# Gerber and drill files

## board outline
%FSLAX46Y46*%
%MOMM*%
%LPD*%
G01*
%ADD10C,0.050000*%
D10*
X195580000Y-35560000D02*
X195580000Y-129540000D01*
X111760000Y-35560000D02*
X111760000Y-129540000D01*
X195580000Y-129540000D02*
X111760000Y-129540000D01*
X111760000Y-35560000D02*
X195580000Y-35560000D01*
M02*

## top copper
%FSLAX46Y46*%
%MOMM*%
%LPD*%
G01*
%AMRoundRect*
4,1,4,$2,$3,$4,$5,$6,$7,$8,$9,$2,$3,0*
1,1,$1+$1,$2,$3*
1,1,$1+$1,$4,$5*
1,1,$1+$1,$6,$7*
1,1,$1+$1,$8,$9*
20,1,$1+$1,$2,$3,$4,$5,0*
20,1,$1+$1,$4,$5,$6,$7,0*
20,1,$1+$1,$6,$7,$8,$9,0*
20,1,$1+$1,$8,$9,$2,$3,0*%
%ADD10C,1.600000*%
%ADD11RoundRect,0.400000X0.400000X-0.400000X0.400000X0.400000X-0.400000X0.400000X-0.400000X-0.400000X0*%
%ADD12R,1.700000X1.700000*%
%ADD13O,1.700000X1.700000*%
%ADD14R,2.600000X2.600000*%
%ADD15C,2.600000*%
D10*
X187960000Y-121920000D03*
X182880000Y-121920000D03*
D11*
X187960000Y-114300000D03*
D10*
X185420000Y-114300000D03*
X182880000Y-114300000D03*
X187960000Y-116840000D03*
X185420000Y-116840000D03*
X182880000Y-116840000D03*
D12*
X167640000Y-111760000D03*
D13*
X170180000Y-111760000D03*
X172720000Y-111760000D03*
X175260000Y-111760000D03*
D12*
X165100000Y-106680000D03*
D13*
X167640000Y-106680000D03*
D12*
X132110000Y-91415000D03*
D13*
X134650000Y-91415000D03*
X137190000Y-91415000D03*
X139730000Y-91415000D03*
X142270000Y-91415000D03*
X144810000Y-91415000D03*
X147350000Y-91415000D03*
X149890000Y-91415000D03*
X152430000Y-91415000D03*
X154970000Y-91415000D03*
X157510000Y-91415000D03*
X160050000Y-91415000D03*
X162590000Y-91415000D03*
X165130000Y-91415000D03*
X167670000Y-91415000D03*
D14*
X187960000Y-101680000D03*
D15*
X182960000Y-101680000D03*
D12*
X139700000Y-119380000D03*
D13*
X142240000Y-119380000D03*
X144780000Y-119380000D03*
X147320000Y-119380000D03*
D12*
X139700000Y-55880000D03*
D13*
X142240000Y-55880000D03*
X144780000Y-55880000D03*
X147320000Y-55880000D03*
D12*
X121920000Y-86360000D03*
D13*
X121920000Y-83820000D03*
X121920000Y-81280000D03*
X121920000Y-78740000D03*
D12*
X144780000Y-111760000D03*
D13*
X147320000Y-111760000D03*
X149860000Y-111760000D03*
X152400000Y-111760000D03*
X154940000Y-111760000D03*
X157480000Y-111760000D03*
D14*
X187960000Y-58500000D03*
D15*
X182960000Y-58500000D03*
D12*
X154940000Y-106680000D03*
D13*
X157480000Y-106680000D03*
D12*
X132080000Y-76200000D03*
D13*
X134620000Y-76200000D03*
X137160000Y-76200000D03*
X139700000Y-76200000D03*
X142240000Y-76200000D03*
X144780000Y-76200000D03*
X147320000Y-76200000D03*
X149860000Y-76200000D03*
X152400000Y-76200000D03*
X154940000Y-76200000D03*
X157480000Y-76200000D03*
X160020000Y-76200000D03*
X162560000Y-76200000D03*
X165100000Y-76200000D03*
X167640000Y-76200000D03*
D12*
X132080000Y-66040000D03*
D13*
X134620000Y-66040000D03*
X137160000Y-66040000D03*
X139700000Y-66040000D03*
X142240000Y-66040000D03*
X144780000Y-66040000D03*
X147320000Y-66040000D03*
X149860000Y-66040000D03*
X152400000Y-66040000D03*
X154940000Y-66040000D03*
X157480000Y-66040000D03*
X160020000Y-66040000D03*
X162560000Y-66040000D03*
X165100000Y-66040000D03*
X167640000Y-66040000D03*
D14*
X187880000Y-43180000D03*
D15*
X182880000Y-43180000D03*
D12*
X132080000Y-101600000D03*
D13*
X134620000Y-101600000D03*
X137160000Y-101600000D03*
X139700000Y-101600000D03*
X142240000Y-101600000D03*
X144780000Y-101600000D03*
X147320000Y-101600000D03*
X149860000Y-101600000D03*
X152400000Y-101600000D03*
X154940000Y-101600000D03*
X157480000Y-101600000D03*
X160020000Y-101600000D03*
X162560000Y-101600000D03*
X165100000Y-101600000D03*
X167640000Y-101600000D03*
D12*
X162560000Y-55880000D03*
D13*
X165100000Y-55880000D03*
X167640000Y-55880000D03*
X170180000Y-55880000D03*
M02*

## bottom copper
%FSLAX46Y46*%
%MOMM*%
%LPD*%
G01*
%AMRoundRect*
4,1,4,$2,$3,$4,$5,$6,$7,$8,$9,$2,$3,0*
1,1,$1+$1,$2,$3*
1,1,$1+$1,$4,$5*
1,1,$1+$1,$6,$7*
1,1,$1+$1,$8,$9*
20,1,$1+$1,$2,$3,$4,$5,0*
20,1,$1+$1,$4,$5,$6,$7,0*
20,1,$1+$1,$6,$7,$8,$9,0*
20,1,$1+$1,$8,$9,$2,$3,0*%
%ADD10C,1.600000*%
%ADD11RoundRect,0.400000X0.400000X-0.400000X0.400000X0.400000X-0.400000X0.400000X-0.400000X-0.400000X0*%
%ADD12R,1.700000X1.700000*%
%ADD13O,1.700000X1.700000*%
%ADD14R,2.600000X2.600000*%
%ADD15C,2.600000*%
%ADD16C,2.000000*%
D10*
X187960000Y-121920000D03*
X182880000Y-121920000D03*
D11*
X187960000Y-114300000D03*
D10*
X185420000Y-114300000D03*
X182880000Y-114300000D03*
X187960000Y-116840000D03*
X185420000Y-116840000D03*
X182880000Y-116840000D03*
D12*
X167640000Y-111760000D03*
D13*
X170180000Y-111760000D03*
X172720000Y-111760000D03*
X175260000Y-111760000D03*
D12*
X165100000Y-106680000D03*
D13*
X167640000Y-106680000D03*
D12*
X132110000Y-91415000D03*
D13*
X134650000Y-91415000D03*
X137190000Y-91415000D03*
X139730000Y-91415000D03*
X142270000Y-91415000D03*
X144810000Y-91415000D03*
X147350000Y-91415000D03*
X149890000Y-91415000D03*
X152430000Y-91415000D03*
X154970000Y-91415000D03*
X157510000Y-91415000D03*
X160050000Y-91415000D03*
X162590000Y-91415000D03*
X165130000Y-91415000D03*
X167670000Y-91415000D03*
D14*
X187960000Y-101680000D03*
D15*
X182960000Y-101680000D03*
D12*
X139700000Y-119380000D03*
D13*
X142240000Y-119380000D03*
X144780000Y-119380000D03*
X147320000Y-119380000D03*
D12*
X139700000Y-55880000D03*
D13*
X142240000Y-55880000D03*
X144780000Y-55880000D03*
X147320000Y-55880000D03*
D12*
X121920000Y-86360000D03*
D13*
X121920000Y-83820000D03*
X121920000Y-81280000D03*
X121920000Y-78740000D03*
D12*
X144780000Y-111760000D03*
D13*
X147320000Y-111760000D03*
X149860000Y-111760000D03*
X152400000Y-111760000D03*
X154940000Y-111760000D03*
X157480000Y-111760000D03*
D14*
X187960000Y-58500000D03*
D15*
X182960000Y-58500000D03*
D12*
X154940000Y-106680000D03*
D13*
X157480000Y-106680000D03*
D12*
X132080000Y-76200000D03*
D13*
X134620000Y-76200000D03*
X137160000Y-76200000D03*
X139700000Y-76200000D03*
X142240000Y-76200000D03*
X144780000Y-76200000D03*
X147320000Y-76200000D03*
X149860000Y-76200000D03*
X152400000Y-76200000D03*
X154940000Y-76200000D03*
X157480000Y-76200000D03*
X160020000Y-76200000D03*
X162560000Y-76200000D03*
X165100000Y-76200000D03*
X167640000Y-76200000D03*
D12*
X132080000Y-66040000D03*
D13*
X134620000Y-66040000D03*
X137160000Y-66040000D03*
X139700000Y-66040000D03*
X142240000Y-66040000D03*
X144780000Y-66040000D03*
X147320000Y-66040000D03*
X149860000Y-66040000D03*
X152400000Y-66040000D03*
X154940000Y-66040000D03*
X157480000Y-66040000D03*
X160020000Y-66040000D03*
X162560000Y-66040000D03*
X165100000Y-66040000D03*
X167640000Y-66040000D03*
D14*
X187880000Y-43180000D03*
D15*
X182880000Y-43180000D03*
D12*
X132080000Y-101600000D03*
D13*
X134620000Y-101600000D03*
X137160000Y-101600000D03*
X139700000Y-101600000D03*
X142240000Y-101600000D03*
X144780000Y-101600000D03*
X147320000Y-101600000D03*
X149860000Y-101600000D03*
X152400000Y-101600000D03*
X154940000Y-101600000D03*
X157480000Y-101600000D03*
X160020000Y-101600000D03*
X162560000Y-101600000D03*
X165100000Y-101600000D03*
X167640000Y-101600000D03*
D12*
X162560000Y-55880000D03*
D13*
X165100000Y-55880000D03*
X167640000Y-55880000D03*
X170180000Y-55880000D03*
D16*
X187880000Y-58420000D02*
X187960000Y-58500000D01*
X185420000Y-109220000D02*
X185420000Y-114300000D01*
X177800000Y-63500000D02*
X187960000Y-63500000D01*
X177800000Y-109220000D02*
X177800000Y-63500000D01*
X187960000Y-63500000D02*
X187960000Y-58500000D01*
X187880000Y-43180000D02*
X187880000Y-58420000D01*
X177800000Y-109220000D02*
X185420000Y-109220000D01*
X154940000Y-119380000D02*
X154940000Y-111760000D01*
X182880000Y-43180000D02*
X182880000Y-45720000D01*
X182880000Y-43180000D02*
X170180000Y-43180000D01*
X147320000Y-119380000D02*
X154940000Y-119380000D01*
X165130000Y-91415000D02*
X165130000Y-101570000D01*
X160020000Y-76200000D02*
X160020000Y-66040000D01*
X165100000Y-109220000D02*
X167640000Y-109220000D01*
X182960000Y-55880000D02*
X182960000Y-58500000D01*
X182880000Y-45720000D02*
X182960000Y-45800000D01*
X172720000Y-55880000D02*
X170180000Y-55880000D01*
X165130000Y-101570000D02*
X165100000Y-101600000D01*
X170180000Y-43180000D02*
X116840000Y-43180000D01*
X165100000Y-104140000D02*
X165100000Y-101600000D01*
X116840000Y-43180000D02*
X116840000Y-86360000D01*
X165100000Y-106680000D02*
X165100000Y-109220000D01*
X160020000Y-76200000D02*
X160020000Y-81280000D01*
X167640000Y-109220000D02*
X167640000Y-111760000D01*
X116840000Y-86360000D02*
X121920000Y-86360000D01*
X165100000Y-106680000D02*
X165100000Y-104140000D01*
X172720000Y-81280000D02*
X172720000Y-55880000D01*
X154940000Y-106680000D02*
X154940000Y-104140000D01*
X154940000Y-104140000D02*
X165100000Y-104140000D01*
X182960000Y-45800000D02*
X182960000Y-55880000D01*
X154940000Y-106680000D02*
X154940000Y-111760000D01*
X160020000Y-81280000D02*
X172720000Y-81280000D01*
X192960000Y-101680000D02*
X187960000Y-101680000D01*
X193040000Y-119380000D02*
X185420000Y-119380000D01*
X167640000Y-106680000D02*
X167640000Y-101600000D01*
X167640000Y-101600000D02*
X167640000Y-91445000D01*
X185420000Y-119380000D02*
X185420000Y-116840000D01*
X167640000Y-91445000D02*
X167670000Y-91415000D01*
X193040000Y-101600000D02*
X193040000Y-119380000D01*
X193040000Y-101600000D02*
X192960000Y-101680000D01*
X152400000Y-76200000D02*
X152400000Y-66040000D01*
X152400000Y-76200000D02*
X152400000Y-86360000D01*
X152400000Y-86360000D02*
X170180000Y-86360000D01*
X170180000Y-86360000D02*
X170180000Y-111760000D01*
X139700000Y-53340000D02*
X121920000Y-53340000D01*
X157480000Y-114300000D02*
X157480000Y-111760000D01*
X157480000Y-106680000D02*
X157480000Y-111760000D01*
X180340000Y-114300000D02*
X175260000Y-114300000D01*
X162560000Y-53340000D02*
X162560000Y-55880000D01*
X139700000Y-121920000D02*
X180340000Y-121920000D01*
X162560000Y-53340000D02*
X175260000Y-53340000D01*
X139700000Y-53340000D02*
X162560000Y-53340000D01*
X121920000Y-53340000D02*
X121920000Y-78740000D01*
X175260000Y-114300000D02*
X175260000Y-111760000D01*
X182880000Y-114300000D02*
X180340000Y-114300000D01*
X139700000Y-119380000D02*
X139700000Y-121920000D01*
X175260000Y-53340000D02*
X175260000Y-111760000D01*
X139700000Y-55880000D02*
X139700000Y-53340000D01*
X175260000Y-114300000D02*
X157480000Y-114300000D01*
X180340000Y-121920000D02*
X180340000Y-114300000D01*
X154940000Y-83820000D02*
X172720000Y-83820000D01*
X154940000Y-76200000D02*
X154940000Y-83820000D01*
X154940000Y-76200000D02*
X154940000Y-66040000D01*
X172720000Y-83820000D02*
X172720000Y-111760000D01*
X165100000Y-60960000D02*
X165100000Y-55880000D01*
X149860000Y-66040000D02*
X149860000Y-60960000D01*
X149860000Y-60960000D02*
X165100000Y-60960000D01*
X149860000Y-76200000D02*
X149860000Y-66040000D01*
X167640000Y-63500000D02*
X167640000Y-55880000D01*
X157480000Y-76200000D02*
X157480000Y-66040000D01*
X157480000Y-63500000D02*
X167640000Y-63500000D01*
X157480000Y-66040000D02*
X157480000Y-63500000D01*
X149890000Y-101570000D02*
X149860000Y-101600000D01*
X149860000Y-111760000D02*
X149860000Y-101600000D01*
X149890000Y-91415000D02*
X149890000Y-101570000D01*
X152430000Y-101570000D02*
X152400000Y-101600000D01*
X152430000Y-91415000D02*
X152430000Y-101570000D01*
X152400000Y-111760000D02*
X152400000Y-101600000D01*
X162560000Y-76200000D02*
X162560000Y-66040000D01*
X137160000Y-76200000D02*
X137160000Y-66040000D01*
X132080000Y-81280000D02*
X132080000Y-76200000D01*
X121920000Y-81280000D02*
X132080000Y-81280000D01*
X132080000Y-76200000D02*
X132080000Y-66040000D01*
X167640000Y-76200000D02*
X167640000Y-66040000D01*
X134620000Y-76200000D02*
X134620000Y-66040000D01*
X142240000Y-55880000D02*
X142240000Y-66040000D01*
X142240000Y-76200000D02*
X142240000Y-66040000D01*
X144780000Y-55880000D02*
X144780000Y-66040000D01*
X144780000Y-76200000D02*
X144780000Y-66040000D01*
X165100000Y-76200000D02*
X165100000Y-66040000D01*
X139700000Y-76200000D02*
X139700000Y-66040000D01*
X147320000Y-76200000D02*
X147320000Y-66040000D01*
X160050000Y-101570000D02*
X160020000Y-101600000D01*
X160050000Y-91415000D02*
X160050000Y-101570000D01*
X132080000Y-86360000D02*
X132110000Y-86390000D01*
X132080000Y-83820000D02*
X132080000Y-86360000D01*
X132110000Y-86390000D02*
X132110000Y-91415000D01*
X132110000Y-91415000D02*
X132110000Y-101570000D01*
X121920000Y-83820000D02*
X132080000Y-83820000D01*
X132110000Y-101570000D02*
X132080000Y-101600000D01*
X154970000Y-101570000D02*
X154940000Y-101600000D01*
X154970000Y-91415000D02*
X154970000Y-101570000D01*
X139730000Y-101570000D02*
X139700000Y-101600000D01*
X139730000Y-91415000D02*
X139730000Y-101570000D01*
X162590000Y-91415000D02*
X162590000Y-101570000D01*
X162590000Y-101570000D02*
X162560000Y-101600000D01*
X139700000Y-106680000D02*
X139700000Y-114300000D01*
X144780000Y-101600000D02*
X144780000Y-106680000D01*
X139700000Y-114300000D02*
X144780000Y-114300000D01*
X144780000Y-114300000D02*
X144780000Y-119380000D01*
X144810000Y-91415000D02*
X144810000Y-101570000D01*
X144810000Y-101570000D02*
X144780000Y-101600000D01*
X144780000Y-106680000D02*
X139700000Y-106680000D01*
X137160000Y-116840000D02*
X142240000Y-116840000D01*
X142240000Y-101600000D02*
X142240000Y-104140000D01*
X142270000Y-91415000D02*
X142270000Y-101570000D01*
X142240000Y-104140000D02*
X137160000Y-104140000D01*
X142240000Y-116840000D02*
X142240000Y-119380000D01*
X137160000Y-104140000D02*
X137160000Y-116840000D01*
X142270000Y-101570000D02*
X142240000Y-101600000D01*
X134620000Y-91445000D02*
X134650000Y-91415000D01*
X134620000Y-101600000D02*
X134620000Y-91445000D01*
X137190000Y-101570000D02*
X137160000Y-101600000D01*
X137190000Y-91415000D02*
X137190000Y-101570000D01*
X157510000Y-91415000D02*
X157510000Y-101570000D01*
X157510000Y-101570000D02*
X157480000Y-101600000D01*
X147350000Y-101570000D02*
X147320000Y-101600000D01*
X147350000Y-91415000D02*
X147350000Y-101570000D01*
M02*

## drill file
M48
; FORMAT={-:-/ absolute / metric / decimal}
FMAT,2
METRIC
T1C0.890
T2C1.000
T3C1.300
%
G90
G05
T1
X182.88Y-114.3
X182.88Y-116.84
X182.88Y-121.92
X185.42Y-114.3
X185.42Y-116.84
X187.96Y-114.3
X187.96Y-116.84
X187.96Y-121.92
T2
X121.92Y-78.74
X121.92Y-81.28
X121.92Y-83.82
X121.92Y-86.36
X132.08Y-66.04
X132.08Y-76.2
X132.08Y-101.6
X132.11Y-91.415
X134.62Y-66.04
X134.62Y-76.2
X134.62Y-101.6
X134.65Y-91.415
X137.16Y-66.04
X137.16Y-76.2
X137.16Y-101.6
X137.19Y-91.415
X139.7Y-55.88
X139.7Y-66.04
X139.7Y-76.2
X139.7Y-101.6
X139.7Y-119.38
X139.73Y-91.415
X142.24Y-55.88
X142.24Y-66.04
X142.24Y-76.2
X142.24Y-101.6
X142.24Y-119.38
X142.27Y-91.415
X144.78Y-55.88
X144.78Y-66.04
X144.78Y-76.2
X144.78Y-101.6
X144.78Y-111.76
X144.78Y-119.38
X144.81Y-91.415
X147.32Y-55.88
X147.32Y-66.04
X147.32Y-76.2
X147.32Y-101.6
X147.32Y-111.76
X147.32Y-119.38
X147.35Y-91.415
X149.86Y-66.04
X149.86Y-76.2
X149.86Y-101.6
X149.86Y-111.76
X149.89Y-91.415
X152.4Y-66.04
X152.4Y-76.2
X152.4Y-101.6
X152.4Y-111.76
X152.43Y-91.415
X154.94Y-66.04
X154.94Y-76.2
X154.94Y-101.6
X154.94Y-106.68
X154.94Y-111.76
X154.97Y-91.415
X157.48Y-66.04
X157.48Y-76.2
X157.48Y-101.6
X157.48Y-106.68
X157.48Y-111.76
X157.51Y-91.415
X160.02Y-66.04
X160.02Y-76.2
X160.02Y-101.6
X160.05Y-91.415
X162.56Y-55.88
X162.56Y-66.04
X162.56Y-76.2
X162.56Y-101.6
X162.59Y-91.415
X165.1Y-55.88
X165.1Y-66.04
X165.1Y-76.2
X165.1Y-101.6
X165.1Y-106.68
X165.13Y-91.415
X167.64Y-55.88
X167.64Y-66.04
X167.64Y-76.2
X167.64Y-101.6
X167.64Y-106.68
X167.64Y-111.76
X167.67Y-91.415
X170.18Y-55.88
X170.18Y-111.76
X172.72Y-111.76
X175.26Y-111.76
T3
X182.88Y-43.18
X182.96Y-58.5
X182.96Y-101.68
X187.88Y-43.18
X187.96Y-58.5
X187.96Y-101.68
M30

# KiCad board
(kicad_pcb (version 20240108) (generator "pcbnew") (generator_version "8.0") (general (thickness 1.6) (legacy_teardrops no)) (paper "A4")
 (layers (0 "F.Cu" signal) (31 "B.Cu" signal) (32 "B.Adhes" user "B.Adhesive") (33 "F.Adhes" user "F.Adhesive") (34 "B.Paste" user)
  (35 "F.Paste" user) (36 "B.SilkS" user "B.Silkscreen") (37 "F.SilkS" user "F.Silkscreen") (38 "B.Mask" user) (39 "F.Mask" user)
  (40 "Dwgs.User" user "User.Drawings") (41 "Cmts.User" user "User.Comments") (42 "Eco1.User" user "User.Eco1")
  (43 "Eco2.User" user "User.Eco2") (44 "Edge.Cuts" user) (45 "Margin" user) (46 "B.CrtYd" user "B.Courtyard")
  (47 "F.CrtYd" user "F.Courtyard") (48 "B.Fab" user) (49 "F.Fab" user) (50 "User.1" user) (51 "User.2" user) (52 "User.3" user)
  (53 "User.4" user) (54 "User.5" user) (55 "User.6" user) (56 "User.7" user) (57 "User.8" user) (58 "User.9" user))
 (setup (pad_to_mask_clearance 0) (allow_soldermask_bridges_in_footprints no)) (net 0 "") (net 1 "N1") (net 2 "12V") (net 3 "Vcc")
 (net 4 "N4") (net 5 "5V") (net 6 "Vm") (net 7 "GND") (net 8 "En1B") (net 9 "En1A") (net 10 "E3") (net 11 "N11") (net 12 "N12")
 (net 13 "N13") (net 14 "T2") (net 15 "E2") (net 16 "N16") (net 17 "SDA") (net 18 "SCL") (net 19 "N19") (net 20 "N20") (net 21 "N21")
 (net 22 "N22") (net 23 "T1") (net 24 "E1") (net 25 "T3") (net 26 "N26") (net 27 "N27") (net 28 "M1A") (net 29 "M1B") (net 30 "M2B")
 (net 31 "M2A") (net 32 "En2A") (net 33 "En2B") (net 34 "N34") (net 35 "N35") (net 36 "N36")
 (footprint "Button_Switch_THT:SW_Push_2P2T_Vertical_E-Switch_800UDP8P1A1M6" (layer "F.Cu") (at 187.96 114.3 -90)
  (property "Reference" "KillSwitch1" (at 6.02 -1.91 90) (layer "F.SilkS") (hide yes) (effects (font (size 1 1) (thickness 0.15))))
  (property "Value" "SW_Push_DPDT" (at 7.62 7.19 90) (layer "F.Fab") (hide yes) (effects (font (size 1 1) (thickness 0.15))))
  (pad "" thru_hole circle (at 7.62 0 90) (size 1.6 1.6) (drill 0.89) (layers "*.Cu" "*.Mask") (remove_unused_layers no))
  (pad "" thru_hole circle (at 7.62 5.08 90) (size 1.6 1.6) (drill 0.89) (layers "*.Cu" "*.Mask") (remove_unused_layers no))
  (pad "1" thru_hole roundrect (at 0 0 90) (size 1.6 1.6) (drill 0.89) (layers "*.Cu" "*.Mask") (remove_unused_layers no)
   (roundrect_rratio 0.25) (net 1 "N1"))
  (pad "2" thru_hole circle (at 0 2.54 90) (size 1.6 1.6) (drill 0.89) (layers "*.Cu" "*.Mask") (remove_unused_layers no) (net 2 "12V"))
  (pad "3" thru_hole circle (at 0 5.08 90) (size 1.6 1.6) (drill 0.89) (layers "*.Cu" "*.Mask") (remove_unused_layers no) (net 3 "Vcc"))
  (pad "4" thru_hole circle (at 2.54 0 90) (size 1.6 1.6) (drill 0.89) (layers "*.Cu" "*.Mask") (remove_unused_layers no) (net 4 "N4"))
  (pad "5" thru_hole circle (at 2.54 2.54 90) (size 1.6 1.6) (drill 0.89) (layers "*.Cu" "*.Mask") (remove_unused_layers no) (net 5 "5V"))
  (pad "6" thru_hole circle (at 2.54 5.08 90) (size 1.6 1.6) (drill 0.89) (layers "*.Cu" "*.Mask") (remove_unused_layers no) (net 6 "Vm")))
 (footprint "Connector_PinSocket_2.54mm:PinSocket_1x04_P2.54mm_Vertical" (layer "F.Cu") (at 167.64 111.76 90)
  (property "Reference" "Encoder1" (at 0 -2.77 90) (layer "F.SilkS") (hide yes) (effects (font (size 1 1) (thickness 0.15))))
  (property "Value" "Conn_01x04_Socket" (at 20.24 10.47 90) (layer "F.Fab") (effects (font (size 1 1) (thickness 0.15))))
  (pad "1" thru_hole rect (at 0 0 90) (size 1.7 1.7) (drill 1) (layers "*.Cu" "*.Mask") (remove_unused_layers no) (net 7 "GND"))
  (pad "2" thru_hole oval (at 0 2.54 90) (size 1.7 1.7) (drill 1) (layers "*.Cu" "*.Mask") (remove_unused_layers no) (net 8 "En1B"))
  (pad "3" thru_hole oval (at 0 5.08 90) (size 1.7 1.7) (drill 1) (layers "*.Cu" "*.Mask") (remove_unused_layers no) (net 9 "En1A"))
  (pad "4" thru_hole oval (at 0 7.62 90) (size 1.7 1.7) (drill 1) (layers "*.Cu" "*.Mask") (remove_unused_layers no) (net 3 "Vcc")))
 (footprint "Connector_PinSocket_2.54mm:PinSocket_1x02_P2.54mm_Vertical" (layer "F.Cu") (at 165.1 106.68 90)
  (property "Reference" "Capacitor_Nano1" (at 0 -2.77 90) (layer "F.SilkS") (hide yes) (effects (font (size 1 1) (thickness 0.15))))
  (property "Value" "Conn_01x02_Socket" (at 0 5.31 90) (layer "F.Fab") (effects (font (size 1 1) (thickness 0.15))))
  (pad "1" thru_hole rect (at 0 0 90) (size 1.7 1.7) (drill 1) (layers "*.Cu" "*.Mask") (remove_unused_layers no) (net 7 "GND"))
  (pad "2" thru_hole oval (at 0 2.54 90) (size 1.7 1.7) (drill 1) (layers "*.Cu" "*.Mask") (remove_unused_layers no) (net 5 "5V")))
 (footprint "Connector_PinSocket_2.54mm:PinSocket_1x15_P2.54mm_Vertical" (layer "F.Cu") (at 132.11 91.415 90)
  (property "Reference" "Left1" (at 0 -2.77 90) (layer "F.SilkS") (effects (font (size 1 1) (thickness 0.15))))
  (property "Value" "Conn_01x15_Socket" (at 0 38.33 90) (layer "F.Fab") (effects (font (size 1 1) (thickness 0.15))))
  (pad "1" thru_hole rect (at 0 0 90) (size 1.7 1.7) (drill 1) (layers "*.Cu" "*.Mask") (remove_unused_layers no) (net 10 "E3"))
  (pad "2" thru_hole oval (at 0 2.54 90) (size 1.7 1.7) (drill 1) (layers "*.Cu" "*.Mask") (remove_unused_layers no) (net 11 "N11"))
  (pad "3" thru_hole oval (at 0 5.08 90) (size 1.7 1.7) (drill 1) (layers "*.Cu" "*.Mask") (remove_unused_layers no) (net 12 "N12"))
  (pad "4" thru_hole oval (at 0 7.62 90) (size 1.7 1.7) (drill 1) (layers "*.Cu" "*.Mask") (remove_unused_layers no) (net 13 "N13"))
  (pad "5" thru_hole oval (at 0 10.16 90) (size 1.7 1.7) (drill 1) (layers "*.Cu" "*.Mask") (remove_unused_layers no) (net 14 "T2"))
  (pad "6" thru_hole oval (at 0 12.7 90) (size 1.7 1.7) (drill 1) (layers "*.Cu" "*.Mask") (remove_unused_layers no) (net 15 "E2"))
  (pad "7" thru_hole oval (at 0 15.24 90) (size 1.7 1.7) (drill 1) (layers "*.Cu" "*.Mask") (remove_unused_layers no) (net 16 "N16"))
  (pad "8" thru_hole oval (at 0 17.78 90) (size 1.7 1.7) (drill 1) (layers "*.Cu" "*.Mask") (remove_unused_layers no) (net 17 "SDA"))
  (pad "9" thru_hole oval (at 0 20.32 90) (size 1.7 1.7) (drill 1) (layers "*.Cu" "*.Mask") (remove_unused_layers no) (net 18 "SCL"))
  (pad "10" thru_hole oval (at 0 22.86 90) (size 1.7 1.7) (drill 1) (layers "*.Cu" "*.Mask") (remove_unused_layers no) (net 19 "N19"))
  (pad "11" thru_hole oval (at 0 25.4 90) (size 1.7 1.7) (drill 1) (layers "*.Cu" "*.Mask") (remove_unused_layers no) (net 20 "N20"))
  (pad "12" thru_hole oval (at 0 27.94 90) (size 1.7 1.7) (drill 1) (layers "*.Cu" "*.Mask") (remove_unused_layers no) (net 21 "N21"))
  (pad "13" thru_hole oval (at 0 30.48 90) (size 1.7 1.7) (drill 1) (layers "*.Cu" "*.Mask") (remove_unused_layers no) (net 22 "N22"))
  (pad "14" thru_hole oval (at 0 33.02 90) (size 1.7 1.7) (drill 1) (layers "*.Cu" "*.Mask") (remove_unused_layers no) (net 7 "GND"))
  (pad "15" thru_hole oval (at 0 35.56 90) (size 1.7 1.7) (drill 1) (layers "*.Cu" "*.Mask") (remove_unused_layers no) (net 5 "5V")))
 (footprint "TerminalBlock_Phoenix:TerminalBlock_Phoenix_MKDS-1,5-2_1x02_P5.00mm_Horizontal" (layer "F.Cu") (at 187.96 101.68 180)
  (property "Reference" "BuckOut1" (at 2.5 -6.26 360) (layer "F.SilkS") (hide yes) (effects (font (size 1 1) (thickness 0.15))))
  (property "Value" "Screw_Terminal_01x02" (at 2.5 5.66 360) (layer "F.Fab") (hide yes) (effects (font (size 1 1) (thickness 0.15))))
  (pad "1" thru_hole rect (at 0 0 180) (size 2.6 2.6) (drill 1.3) (layers "*.Cu" "*.Mask") (remove_unused_layers no) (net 5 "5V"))
  (pad "2" thru_hole circle (at 5 0 180) (size 2.6 2.6) (drill 1.3) (layers "*.Cu" "*.Mask") (remove_unused_layers no) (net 7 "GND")))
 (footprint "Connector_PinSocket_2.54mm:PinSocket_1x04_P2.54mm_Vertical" (layer "F.Cu") (at 139.7 119.38 90)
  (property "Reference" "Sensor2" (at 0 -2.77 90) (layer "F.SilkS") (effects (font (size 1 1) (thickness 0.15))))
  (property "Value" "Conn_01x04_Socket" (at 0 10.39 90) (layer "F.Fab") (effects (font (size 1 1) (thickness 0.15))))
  (pad "1" thru_hole rect (at 0 0 90) (size 1.7 1.7) (drill 1) (layers "*.Cu" "*.Mask") (remove_unused_layers no) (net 3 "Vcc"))
  (pad "2" thru_hole oval (at 0 2.54 90) (size 1.7 1.7) (drill 1) (layers "*.Cu" "*.Mask") (remove_unused_layers no) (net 14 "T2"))
  (pad "3" thru_hole oval (at 0 5.08 90) (size 1.7 1.7) (drill 1) (layers "*.Cu" "*.Mask") (remove_unused_layers no) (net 15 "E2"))
  (pad "4" thru_hole oval (at 0 7.62 90) (size 1.7 1.7) (drill 1) (layers "*.Cu" "*.Mask") (remove_unused_layers no) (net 7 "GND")))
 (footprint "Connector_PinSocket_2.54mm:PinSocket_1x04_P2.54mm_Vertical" (layer "F.Cu") (at 139.7 55.88 90)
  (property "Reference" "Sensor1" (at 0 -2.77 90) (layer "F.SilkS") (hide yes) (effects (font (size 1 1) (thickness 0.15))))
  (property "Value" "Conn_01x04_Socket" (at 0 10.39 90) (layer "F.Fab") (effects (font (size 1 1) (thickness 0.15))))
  (pad "1" thru_hole rect (at 0 0 90) (size 1.7 1.7) (drill 1) (layers "*.Cu" "*.Mask") (remove_unused_layers no) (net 3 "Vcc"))
  (pad "2" thru_hole oval (at 0 2.54 90) (size 1.7 1.7) (drill 1) (layers "*.Cu" "*.Mask") (remove_unused_layers no) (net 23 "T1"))
  (pad "3" thru_hole oval (at 0 5.08 90) (size 1.7 1.7) (drill 1) (layers "*.Cu" "*.Mask") (remove_unused_layers no) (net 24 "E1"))
  (pad "4" thru_hole oval (at 0 7.62 90) (size 1.7 1.7) (drill 1) (layers "*.Cu" "*.Mask") (remove_unused_layers no) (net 7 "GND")))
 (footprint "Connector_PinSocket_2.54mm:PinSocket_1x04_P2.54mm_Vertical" (layer "F.Cu") (at 121.92 86.36 180)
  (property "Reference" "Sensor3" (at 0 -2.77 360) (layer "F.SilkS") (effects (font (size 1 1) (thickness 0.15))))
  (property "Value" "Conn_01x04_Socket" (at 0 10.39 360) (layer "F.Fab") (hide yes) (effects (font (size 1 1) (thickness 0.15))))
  (pad "1" thru_hole rect (at 0 0 180) (size 1.7 1.7) (drill 1) (layers "*.Cu" "*.Mask") (remove_unused_layers no) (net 7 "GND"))
  (pad "2" thru_hole oval (at 0 2.54 180) (size 1.7 1.7) (drill 1) (layers "*.Cu" "*.Mask") (remove_unused_layers no) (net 10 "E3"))
  (pad "3" thru_hole oval (at 0 5.08 180) (size 1.7 1.7) (drill 1) (layers "*.Cu" "*.Mask") (remove_unused_layers no) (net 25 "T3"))
  (pad "4" thru_hole oval (at 0 7.62 180) (size 1.7 1.7) (drill 1) (layers "*.Cu" "*.Mask") (remove_unused_layers no) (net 3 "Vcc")))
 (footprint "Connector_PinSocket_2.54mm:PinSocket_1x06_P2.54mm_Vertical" (layer "F.Cu") (at 144.78 111.76 90)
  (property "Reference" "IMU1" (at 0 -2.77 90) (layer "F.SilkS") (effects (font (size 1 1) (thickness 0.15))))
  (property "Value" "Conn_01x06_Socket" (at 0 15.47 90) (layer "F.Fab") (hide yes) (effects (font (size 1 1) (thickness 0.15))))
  (pad "1" thru_hole rect (at 0 0 90) (size 1.7 1.7) (drill 1) (layers "*.Cu" "*.Mask") (remove_unused_layers no) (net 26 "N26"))
  (pad "2" thru_hole oval (at 0 2.54 90) (size 1.7 1.7) (drill 1) (layers "*.Cu" "*.Mask") (remove_unused_layers no) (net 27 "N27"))
  (pad "3" thru_hole oval (at 0 5.08 90) (size 1.7 1.7) (drill 1) (layers "*.Cu" "*.Mask") (remove_unused_layers no) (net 17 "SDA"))
  (pad "4" thru_hole oval (at 0 7.62 90) (size 1.7 1.7) (drill 1) (layers "*.Cu" "*.Mask") (remove_unused_layers no) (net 18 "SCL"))
  (pad "5" thru_hole oval (at 0 10.16 90) (size 1.7 1.7) (drill 1) (layers "*.Cu" "*.Mask") (remove_unused_layers no) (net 7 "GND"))
  (pad "6" thru_hole oval (at 0 12.7 90) (size 1.7 1.7) (drill 1) (layers "*.Cu" "*.Mask") (remove_unused_layers no) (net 3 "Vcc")))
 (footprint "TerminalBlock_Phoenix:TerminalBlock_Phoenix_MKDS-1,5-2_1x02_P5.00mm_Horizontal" (layer "F.Cu") (at 187.96 58.5 180)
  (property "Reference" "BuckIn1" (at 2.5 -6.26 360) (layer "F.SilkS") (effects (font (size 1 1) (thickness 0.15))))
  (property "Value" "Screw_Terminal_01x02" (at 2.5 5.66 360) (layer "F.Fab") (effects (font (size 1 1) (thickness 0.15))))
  (pad "1" thru_hole rect (at 0 0 180) (size 2.6 2.6) (drill 1.3) (layers "*.Cu" "*.Mask") (remove_unused_layers no) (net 2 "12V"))
  (pad "2" thru_hole circle (at 5 0 180) (size 2.6 2.6) (drill 1.3) (layers "*.Cu" "*.Mask") (remove_unused_layers no) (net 7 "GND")))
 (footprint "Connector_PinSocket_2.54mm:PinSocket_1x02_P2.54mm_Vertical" (layer "F.Cu") (at 154.94 106.68 90)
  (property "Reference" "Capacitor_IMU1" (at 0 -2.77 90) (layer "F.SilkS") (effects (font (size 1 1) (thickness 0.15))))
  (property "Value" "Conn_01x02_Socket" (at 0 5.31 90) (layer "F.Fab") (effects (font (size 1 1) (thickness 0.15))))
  (pad "1" thru_hole rect (at 0 0 90) (size 1.7 1.7) (drill 1) (layers "*.Cu" "*.Mask") (remove_unused_layers no) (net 7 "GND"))
  (pad "2" thru_hole oval (at 0 2.54 90) (size 1.7 1.7) (drill 1) (layers "*.Cu" "*.Mask") (remove_unused_layers no) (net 3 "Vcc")))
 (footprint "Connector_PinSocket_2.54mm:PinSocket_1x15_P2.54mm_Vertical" (layer "F.Cu") (at 132.08 76.2 90)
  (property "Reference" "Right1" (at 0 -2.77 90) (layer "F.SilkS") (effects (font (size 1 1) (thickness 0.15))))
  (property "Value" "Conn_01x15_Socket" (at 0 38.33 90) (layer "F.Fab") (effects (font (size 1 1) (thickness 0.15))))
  (pad "1" thru_hole rect (at 0 0 90) (size 1.7 1.7) (drill 1) (layers "*.Cu" "*.Mask") (remove_unused_layers no) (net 25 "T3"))
  (pad "2" thru_hole oval (at 0 2.54 90) (size 1.7 1.7) (drill 1) (layers "*.Cu" "*.Mask") (remove_unused_layers no) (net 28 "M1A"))
  (pad "3" thru_hole oval (at 0 5.08 90) (size 1.7 1.7) (drill 1) (layers "*.Cu" "*.Mask") (remove_unused_layers no) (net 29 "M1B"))
  (pad "4" thru_hole oval (at 0 7.62 90) (size 1.7 1.7) (drill 1) (layers "*.Cu" "*.Mask") (remove_unused_layers no) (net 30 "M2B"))
  (pad "5" thru_hole oval (at 0 10.16 90) (size 1.7 1.7) (drill 1) (layers "*.Cu" "*.Mask") (remove_unused_layers no) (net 23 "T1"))
  (pad "6" thru_hole oval (at 0 12.7 90) (size 1.7 1.7) (drill 1) (layers "*.Cu" "*.Mask") (remove_unused_layers no) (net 24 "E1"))
  (pad "7" thru_hole oval (at 0 15.24 90) (size 1.7 1.7) (drill 1) (layers "*.Cu" "*.Mask") (remove_unused_layers no) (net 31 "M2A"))
  (pad "8" thru_hole oval (at 0 17.78 90) (size 1.7 1.7) (drill 1) (layers "*.Cu" "*.Mask") (remove_unused_layers no) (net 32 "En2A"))
  (pad "9" thru_hole oval (at 0 20.32 90) (size 1.7 1.7) (drill 1) (layers "*.Cu" "*.Mask") (remove_unused_layers no) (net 8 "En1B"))
  (pad "10" thru_hole oval (at 0 22.86 90) (size 1.7 1.7) (drill 1) (layers "*.Cu" "*.Mask") (remove_unused_layers no) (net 9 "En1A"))
  (pad "11" thru_hole oval (at 0 25.4 90) (size 1.7 1.7) (drill 1) (layers "*.Cu" "*.Mask") (remove_unused_layers no) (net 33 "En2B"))
  (pad "12" thru_hole oval (at 0 27.94 90) (size 1.7 1.7) (drill 1) (layers "*.Cu" "*.Mask") (remove_unused_layers no) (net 7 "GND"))
  (pad "13" thru_hole oval (at 0 30.48 90) (size 1.7 1.7) (drill 1) (layers "*.Cu" "*.Mask") (remove_unused_layers no) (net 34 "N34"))
  (pad "14" thru_hole oval (at 0 33.02 90) (size 1.7 1.7) (drill 1) (layers "*.Cu" "*.Mask") (remove_unused_layers no) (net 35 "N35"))
  (pad "15" thru_hole oval (at 0 35.56 90) (size 1.7 1.7) (drill 1) (layers "*.Cu" "*.Mask") (remove_unused_layers no) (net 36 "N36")))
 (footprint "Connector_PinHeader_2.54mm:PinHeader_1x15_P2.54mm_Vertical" (layer "F.Cu") (at 132.08 66.04 90)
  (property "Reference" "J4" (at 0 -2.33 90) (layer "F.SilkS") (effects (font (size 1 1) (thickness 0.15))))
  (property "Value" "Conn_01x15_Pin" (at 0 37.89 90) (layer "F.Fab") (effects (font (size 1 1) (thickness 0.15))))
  (pad "1" thru_hole rect (at 0 0 90) (size 1.7 1.7) (drill 1) (layers "*.Cu" "*.Mask") (remove_unused_layers no) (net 25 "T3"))
  (pad "2" thru_hole oval (at 0 2.54 90) (size 1.7 1.7) (drill 1) (layers "*.Cu" "*.Mask") (remove_unused_layers no) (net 28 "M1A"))
  (pad "3" thru_hole oval (at 0 5.08 90) (size 1.7 1.7) (drill 1) (layers "*.Cu" "*.Mask") (remove_unused_layers no) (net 29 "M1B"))
  (pad "4" thru_hole oval (at 0 7.62 90) (size 1.7 1.7) (drill 1) (layers "*.Cu" "*.Mask") (remove_unused_layers no) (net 30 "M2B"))
  (pad "5" thru_hole oval (at 0 10.16 90) (size 1.7 1.7) (drill 1) (layers "*.Cu" "*.Mask") (remove_unused_layers no) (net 23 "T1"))
  (pad "6" thru_hole oval (at 0 12.7 90) (size 1.7 1.7) (drill 1) (layers "*.Cu" "*.Mask") (remove_unused_layers no) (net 24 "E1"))
  (pad "7" thru_hole oval (at 0 15.24 90) (size 1.7 1.7) (drill 1) (layers "*.Cu" "*.Mask") (remove_unused_layers no) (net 31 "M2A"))
  (pad "8" thru_hole oval (at 0 17.78 90) (size 1.7 1.7) (drill 1) (layers "*.Cu" "*.Mask") (remove_unused_layers no) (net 32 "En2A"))
  (pad "9" thru_hole oval (at 0 20.32 90) (size 1.7 1.7) (drill 1) (layers "*.Cu" "*.Mask") (remove_unused_layers no) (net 8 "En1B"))
  (pad "10" thru_hole oval (at 0 22.86 90) (size 1.7 1.7) (drill 1) (layers "*.Cu" "*.Mask") (remove_unused_layers no) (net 9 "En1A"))
  (pad "11" thru_hole oval (at 0 25.4 90) (size 1.7 1.7) (drill 1) (layers "*.Cu" "*.Mask") (remove_unused_layers no) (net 33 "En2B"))
  (pad "12" thru_hole oval (at 0 27.94 90) (size 1.7 1.7) (drill 1) (layers "*.Cu" "*.Mask") (remove_unused_layers no) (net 7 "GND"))
  (pad "13" thru_hole oval (at 0 30.48 90) (size 1.7 1.7) (drill 1) (layers "*.Cu" "*.Mask") (remove_unused_layers no) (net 34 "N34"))
  (pad "14" thru_hole oval (at 0 33.02 90) (size 1.7 1.7) (drill 1) (layers "*.Cu" "*.Mask") (remove_unused_layers no) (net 35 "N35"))
  (pad "15" thru_hole oval (at 0 35.56 90) (size 1.7 1.7) (drill 1) (layers "*.Cu" "*.Mask") (remove_unused_layers no) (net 36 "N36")))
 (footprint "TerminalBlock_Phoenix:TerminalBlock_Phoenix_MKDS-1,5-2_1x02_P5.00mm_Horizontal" (layer "F.Cu") (at 187.88 43.18 180)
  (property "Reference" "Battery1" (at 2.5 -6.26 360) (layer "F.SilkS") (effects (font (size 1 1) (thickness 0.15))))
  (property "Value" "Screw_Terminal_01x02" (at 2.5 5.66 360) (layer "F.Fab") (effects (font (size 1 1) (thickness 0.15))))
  (pad "1" thru_hole rect (at 0 0 180) (size 2.6 2.6) (drill 1.3) (layers "*.Cu" "*.Mask") (remove_unused_layers no) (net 2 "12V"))
  (pad "2" thru_hole circle (at 5 0 180) (size 2.6 2.6) (drill 1.3) (layers "*.Cu" "*.Mask") (remove_unused_layers no) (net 7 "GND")))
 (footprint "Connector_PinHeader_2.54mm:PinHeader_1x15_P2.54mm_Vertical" (layer "F.Cu") (at 132.08 101.6 90)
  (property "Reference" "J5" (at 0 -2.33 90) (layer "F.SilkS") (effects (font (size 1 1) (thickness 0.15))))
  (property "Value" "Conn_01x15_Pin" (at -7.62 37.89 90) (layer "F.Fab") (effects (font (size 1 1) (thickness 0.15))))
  (pad "1" thru_hole rect (at 0 0 90) (size 1.7 1.7) (drill 1) (layers "*.Cu" "*.Mask") (remove_unused_layers no) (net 10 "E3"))
  (pad "2" thru_hole oval (at 0 2.54 90) (size 1.7 1.7) (drill 1) (layers "*.Cu" "*.Mask") (remove_unused_layers no) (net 11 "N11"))
  (pad "3" thru_hole oval (at 0 5.08 90) (size 1.7 1.7) (drill 1) (layers "*.Cu" "*.Mask") (remove_unused_layers no) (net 12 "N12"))
  (pad "4" thru_hole oval (at 0 7.62 90) (size 1.7 1.7) (drill 1) (layers "*.Cu" "*.Mask") (remove_unused_layers no) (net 13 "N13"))
  (pad "5" thru_hole oval (at 0 10.16 90) (size 1.7 1.7) (drill 1) (layers "*.Cu" "*.Mask") (remove_unused_layers no) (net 14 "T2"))
  (pad "6" thru_hole oval (at 0 12.7 90) (size 1.7 1.7) (drill 1) (layers "*.Cu" "*.Mask") (remove_unused_layers no) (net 15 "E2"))
  (pad "7" thru_hole oval (at 0 15.24 90) (size 1.7 1.7) (drill 1) (layers "*.Cu" "*.Mask") (remove_unused_layers no) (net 16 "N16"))
  (pad "8" thru_hole oval (at 0 17.78 90) (size 1.7 1.7) (drill 1) (layers "*.Cu" "*.Mask") (remove_unused_layers no) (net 17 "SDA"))
  (pad "9" thru_hole oval (at 0 20.32 90) (size 1.7 1.7) (drill 1) (layers "*.Cu" "*.Mask") (remove_unused_layers no) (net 18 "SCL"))
  (pad "10" thru_hole oval (at 0 22.86 90) (size 1.7 1.7) (drill 1) (layers "*.Cu" "*.Mask") (remove_unused_layers no) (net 19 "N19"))
  (pad "11" thru_hole oval (at 0 25.4 90) (size 1.7 1.7) (drill 1) (layers "*.Cu" "*.Mask") (remove_unused_layers no) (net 20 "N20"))
  (pad "12" thru_hole oval (at 0 27.94 90) (size 1.7 1.7) (drill 1) (layers "*.Cu" "*.Mask") (remove_unused_layers no) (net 21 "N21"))
  (pad "13" thru_hole oval (at 0 30.48 90) (size 1.7 1.7) (drill 1) (layers "*.Cu" "*.Mask") (remove_unused_layers no) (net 22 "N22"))
  (pad "14" thru_hole oval (at 0 33.02 90) (size 1.7 1.7) (drill 1) (layers "*.Cu" "*.Mask") (remove_unused_layers no) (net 7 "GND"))
  (pad "15" thru_hole oval (at 0 35.56 90) (size 1.7 1.7) (drill 1) (layers "*.Cu" "*.Mask") (remove_unused_layers no) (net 5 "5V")))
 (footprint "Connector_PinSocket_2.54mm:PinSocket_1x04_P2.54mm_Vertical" (layer "F.Cu") (at 162.56 55.88 90)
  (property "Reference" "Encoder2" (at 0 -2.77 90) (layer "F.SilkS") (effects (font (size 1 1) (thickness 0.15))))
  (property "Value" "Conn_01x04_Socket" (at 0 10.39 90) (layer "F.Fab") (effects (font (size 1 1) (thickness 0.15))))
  (pad "1" thru_hole rect (at 0 0 90) (size 1.7 1.7) (drill 1) (layers "*.Cu" "*.Mask") (remove_unused_layers no) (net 3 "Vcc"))
  (pad "2" thru_hole oval (at 0 2.54 90) (size 1.7 1.7) (drill 1) (layers "*.Cu" "*.Mask") (remove_unused_layers no) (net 32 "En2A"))
  (pad "3" thru_hole oval (at 0 5.08 90) (size 1.7 1.7) (drill 1) (layers "*.Cu" "*.Mask") (remove_unused_layers no) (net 33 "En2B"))
  (pad "4" thru_hole oval (at 0 7.62 90) (size 1.7 1.7) (drill 1) (layers "*.Cu" "*.Mask") (remove_unused_layers no) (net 7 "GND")))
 (gr_line (start 195.58 35.56) (end 195.58 129.54) (stroke (width 0.05) (type default)) (layer "Edge.Cuts"))
 (gr_line (start 111.76 35.56) (end 111.76 129.54) (stroke (width 0.05) (type default)) (layer "Edge.Cuts"))
 (gr_line (start 195.58 129.54) (end 111.76 129.54) (stroke (width 0.05) (type default)) (layer "Edge.Cuts"))
 (gr_line (start 111.76 35.56) (end 195.58 35.56) (stroke (width 0.05) (type default)) (layer "Edge.Cuts"))
 (segment (start 187.88 58.42) (end 187.96 58.5) (width 2) (layer "B.Cu") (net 2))
 (segment (start 185.42 109.22) (end 185.42 114.3) (width 2) (layer "B.Cu") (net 2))
 (segment (start 177.8 63.5) (end 187.96 63.5) (width 2) (layer "B.Cu") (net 2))
 (segment (start 177.8 109.22) (end 177.8 63.5) (width 2) (layer "B.Cu") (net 2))
 (segment (start 187.96 63.5) (end 187.96 58.5) (width 2) (layer "B.Cu") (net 2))
 (segment (start 187.88 43.18) (end 187.88 58.42) (width 2) (layer "B.Cu") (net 2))
 (segment (start 177.8 109.22) (end 185.42 109.22) (width 2) (layer "B.Cu") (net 2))
 (segment (start 154.94 119.38) (end 154.94 111.76) (width 2) (layer "B.Cu") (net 7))
 (segment (start 182.88 43.18) (end 182.88 45.72) (width 2) (layer "B.Cu") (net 7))
 (segment (start 182.88 43.18) (end 170.18 43.18) (width 2) (layer "B.Cu") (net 7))
 (segment (start 147.32 119.38) (end 154.94 119.38) (width 2) (layer "B.Cu") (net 7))
 (segment (start 165.13 91.415) (end 165.13 101.57) (width 2) (layer "B.Cu") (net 7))
 (segment (start 160.02 76.2) (end 160.02 66.04) (width 2) (layer "B.Cu") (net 7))
 (segment (start 165.1 109.22) (end 167.64 109.22) (width 2) (layer "B.Cu") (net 7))
 (segment (start 182.96 55.88) (end 182.96 58.5) (width 2) (layer "B.Cu") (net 7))
 (segment (start 182.88 45.72) (end 182.96 45.8) (width 2) (layer "B.Cu") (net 7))
 (segment (start 172.72 55.88) (end 170.18 55.88) (width 2) (layer "B.Cu") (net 7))
 (segment (start 165.13 101.57) (end 165.1 101.6) (width 2) (layer "B.Cu") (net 7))
 (segment (start 170.18 43.18) (end 116.84 43.18) (width 2) (layer "B.Cu") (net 7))
 (segment (start 165.1 104.14) (end 165.1 101.6) (width 2) (layer "B.Cu") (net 7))
 (segment (start 116.84 43.18) (end 116.84 86.36) (width 2) (layer "B.Cu") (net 7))
 (segment (start 165.1 106.68) (end 165.1 109.22) (width 2) (layer "B.Cu") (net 7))
 (segment (start 160.02 76.2) (end 160.02 81.28) (width 2) (layer "B.Cu") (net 7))
 (segment (start 167.64 109.22) (end 167.64 111.76) (width 2) (layer "B.Cu") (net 7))
 (segment (start 116.84 86.36) (end 121.92 86.36) (width 2) (layer "B.Cu") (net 7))
 (segment (start 165.1 106.68) (end 165.1 104.14) (width 2) (layer "B.Cu") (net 7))
 (segment (start 172.72 81.28) (end 172.72 55.88) (width 2) (layer "B.Cu") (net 7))
 (segment (start 154.94 106.68) (end 154.94 104.14) (width 2) (layer "B.Cu") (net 7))
 (segment (start 154.94 104.14) (end 165.1 104.14) (width 2) (layer "B.Cu") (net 7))
 (segment (start 182.96 45.8) (end 182.96 55.88) (width 2) (layer "B.Cu") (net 7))
 (segment (start 154.94 106.68) (end 154.94 111.76) (width 2) (layer "B.Cu") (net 7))
 (segment (start 160.02 81.28) (end 172.72 81.28) (width 2) (layer "B.Cu") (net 7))
 (segment (start 192.96 101.68) (end 187.96 101.68) (width 2) (layer "B.Cu") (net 5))
 (segment (start 193.04 119.38) (end 185.42 119.38) (width 2) (layer "B.Cu") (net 5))
 (segment (start 167.64 106.68) (end 167.64 101.6) (width 2) (layer "B.Cu") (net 5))
 (segment (start 167.64 101.6) (end 167.64 91.445) (width 2) (layer "B.Cu") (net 5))
 (segment (start 185.42 119.38) (end 185.42 116.84) (width 2) (layer "B.Cu") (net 5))
 (segment (start 167.64 91.445) (end 167.67 91.415) (width 2) (layer "B.Cu") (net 5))
 (segment (start 193.04 101.6) (end 193.04 119.38) (width 2) (layer "B.Cu") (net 5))
 (segment (start 193.04 101.6) (end 192.96 101.68) (width 2) (layer "B.Cu") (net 5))
 (segment (start 152.4 76.2) (end 152.4 66.04) (width 2) (layer "B.Cu") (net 8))
 (segment (start 152.4 76.2) (end 152.4 86.36) (width 2) (layer "B.Cu") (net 8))
 (segment (start 152.4 86.36) (end 170.18 86.36) (width 2) (layer "B.Cu") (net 8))
 (segment (start 170.18 86.36) (end 170.18 111.76) (width 2) (layer "B.Cu") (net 8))
 (segment (start 139.7 53.34) (end 121.92 53.34) (width 2) (layer "B.Cu") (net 3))
 (segment (start 157.48 114.3) (end 157.48 111.76) (width 2) (layer "B.Cu") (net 3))
 (segment (start 157.48 106.68) (end 157.48 111.76) (width 2) (layer "B.Cu") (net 3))
 (segment (start 180.34 114.3) (end 175.26 114.3) (width 2) (layer "B.Cu") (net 3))
 (segment (start 162.56 53.34) (end 162.56 55.88) (width 2) (layer "B.Cu") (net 3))
 (segment (start 139.7 121.92) (end 180.34 121.92) (width 2) (layer "B.Cu") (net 3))
 (segment (start 162.56 53.34) (end 175.26 53.34) (width 2) (layer "B.Cu") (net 3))
 (segment (start 139.7 53.34) (end 162.56 53.34) (width 2) (layer "B.Cu") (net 3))
 (segment (start 121.92 53.34) (end 121.92 78.74) (width 2) (layer "B.Cu") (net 3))
 (segment (start 175.26 114.3) (end 175.26 111.76) (width 2) (layer "B.Cu") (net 3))
 (segment (start 182.88 114.3) (end 180.34 114.3) (width 2) (layer "B.Cu") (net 3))
 (segment (start 139.7 119.38) (end 139.7 121.92) (width 2) (layer "B.Cu") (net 3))
 (segment (start 175.26 53.34) (end 175.26 111.76) (width 2) (layer "B.Cu") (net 3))
 (segment (start 139.7 55.88) (end 139.7 53.34) (width 2) (layer "B.Cu") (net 3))
 (segment (start 175.26 114.3) (end 157.48 114.3) (width 2) (layer "B.Cu") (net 3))
 (segment (start 180.34 121.92) (end 180.34 114.3) (width 2) (layer "B.Cu") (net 3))
 (segment (start 154.94 83.82) (end 172.72 83.82) (width 2) (layer "B.Cu") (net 9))
 (segment (start 154.94 76.2) (end 154.94 83.82) (width 2) (layer "B.Cu") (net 9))
 (segment (start 154.94 76.2) (end 154.94 66.04) (width 2) (layer "B.Cu") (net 9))
 (segment (start 172.72 83.82) (end 172.72 111.76) (width 2) (layer "B.Cu") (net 9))
 (segment (start 165.1 60.96) (end 165.1 55.88) (width 2) (layer "B.Cu") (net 32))
 (segment (start 149.86 66.04) (end 149.86 60.96) (width 2) (layer "B.Cu") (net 32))
 (segment (start 149.86 60.96) (end 165.1 60.96) (width 2) (layer "B.Cu") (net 32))
 (segment (start 149.86 76.2) (end 149.86 66.04) (width 2) (layer "B.Cu") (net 32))
 (segment (start 167.64 63.5) (end 167.64 55.88) (width 2) (layer "B.Cu") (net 33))
 (segment (start 157.48 76.2) (end 157.48 66.04) (width 2) (layer "B.Cu") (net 33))
 (segment (start 157.48 63.5) (end 167.64 63.5) (width 2) (layer "B.Cu") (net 33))
 (segment (start 157.48 66.04) (end 157.48 63.5) (width 2) (layer "B.Cu") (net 33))
 (segment (start 149.89 101.57) (end 149.86 101.6) (width 2) (layer "B.Cu") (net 17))
 (segment (start 149.86 111.76) (end 149.86 101.6) (width 2) (layer "B.Cu") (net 17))
 (segment (start 149.89 91.415) (end 149.89 101.57) (width 2) (layer "B.Cu") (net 17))
 (segment (start 152.43 101.57) (end 152.4 101.6) (width 2) (layer "B.Cu") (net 18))
 (segment (start 152.43 91.415) (end 152.43 101.57) (width 2) (layer "B.Cu") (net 18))
 (segment (start 152.4 111.76) (end 152.4 101.6) (width 2) (layer "B.Cu") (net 18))
 (segment (start 162.56 76.2) (end 162.56 66.04) (width 2) (layer "B.Cu") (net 34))
 (segment (start 137.16 76.2) (end 137.16 66.04) (width 2) (layer "B.Cu") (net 29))
 (segment (start 132.08 81.28) (end 132.08 76.2) (width 2) (layer "B.Cu") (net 25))
 (segment (start 121.92 81.28) (end 132.08 81.28) (width 2) (layer "B.Cu") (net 25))
 (segment (start 132.08 76.2) (end 132.08 66.04) (width 2) (layer "B.Cu") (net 25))
 (segment (start 167.64 76.2) (end 167.64 66.04) (width 2) (layer "B.Cu") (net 36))
 (segment (start 134.62 76.2) (end 134.62 66.04) (width 2) (layer "B.Cu") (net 28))
 (segment (start 142.24 55.88) (end 142.24 66.04) (width 2) (layer "B.Cu") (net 23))
 (segment (start 142.24 76.2) (end 142.24 66.04) (width 2) (layer "B.Cu") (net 23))
 (segment (start 144.78 55.88) (end 144.78 66.04) (width 2) (layer "B.Cu") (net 24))
 (segment (start 144.78 76.2) (end 144.78 66.04) (width 2) (layer "B.Cu") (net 24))
 (segment (start 165.1 76.2) (end 165.1 66.04) (width 2) (layer "B.Cu") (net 35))
 (segment (start 139.7 76.2) (end 139.7 66.04) (width 2) (layer "B.Cu") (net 30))
 (segment (start 147.32 76.2) (end 147.32 66.04) (width 2) (layer "B.Cu") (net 31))
 (segment (start 160.05 101.57) (end 160.02 101.6) (width 2) (layer "B.Cu") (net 21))
 (segment (start 160.05 91.415) (end 160.05 101.57) (width 2) (layer "B.Cu") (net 21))
 (segment (start 132.08 86.36) (end 132.11 86.39) (width 2) (layer "B.Cu") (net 10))
 (segment (start 132.08 83.82) (end 132.08 86.36) (width 2) (layer "B.Cu") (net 10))
 (segment (start 132.11 86.39) (end 132.11 91.415) (width 2) (layer "B.Cu") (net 10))
 (segment (start 132.11 91.415) (end 132.11 101.57) (width 2) (layer "B.Cu") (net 10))
 (segment (start 121.92 83.82) (end 132.08 83.82) (width 2) (layer "B.Cu") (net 10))
 (segment (start 132.11 101.57) (end 132.08 101.6) (width 2) (layer "B.Cu") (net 10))
 (segment (start 154.97 101.57) (end 154.94 101.6) (width 2) (layer "B.Cu") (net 19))
 (segment (start 154.97 91.415) (end 154.97 101.57) (width 2) (layer "B.Cu") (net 19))
 (segment (start 139.73 101.57) (end 139.7 101.6) (width 2) (layer "B.Cu") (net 13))
 (segment (start 139.73 91.415) (end 139.73 101.57) (width 2) (layer "B.Cu") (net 13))
 (segment (start 162.59 91.415) (end 162.59 101.57) (width 2) (layer "B.Cu") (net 22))
 (segment (start 162.59 101.57) (end 162.56 101.6) (width 2) (layer "B.Cu") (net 22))
 (segment (start 139.7 106.68) (end 139.7 114.3) (width 2) (layer "B.Cu") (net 15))
 (segment (start 144.78 101.6) (end 144.78 106.68) (width 2) (layer "B.Cu") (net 15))
 (segment (start 139.7 114.3) (end 144.78 114.3) (width 2) (layer "B.Cu") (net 15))
 (segment (start 144.78 114.3) (end 144.78 119.38) (width 2) (layer "B.Cu") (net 15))
 (segment (start 144.81 91.415) (end 144.81 101.57) (width 2) (layer "B.Cu") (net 15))
 (segment (start 144.81 101.57) (end 144.78 101.6) (width 2) (layer "B.Cu") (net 15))
 (segment (start 144.78 106.68) (end 139.7 106.68) (width 2) (layer "B.Cu") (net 15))
 (segment (start 137.16 116.84) (end 142.24 116.84) (width 2) (layer "B.Cu") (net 14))
 (segment (start 142.24 101.6) (end 142.24 104.14) (width 2) (layer "B.Cu") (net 14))
 (segment (start 142.27 91.415) (end 142.27 101.57) (width 2) (layer "B.Cu") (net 14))
 (segment (start 142.24 104.14) (end 137.16 104.14) (width 2) (layer "B.Cu") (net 14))
 (segment (start 142.24 116.84) (end 142.24 119.38) (width 2) (layer "B.Cu") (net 14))
 (segment (start 137.16 104.14) (end 137.16 116.84) (width 2) (layer "B.Cu") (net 14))
 (segment (start 142.27 101.57) (end 142.24 101.6) (width 2) (layer "B.Cu") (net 14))
 (segment (start 134.62 91.445) (end 134.65 91.415) (width 2) (layer "B.Cu") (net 11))
 (segment (start 134.62 101.6) (end 134.62 91.445) (width 2) (layer "B.Cu") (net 11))
 (segment (start 137.19 101.57) (end 137.16 101.6) (width 2) (layer "B.Cu") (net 12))
 (segment (start 137.19 91.415) (end 137.19 101.57) (width 2) (layer "B.Cu") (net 12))
 (segment (start 157.51 91.415) (end 157.51 101.57) (width 2) (layer "B.Cu") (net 20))
 (segment (start 157.51 101.57) (end 157.48 101.6) (width 2) (layer "B.Cu") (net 20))
 (segment (start 147.35 101.57) (end 147.32 101.6) (width 2) (layer "B.Cu") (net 16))
 (segment (start 147.35 91.415) (end 147.35 101.57) (width 2) (layer "B.Cu") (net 16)))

